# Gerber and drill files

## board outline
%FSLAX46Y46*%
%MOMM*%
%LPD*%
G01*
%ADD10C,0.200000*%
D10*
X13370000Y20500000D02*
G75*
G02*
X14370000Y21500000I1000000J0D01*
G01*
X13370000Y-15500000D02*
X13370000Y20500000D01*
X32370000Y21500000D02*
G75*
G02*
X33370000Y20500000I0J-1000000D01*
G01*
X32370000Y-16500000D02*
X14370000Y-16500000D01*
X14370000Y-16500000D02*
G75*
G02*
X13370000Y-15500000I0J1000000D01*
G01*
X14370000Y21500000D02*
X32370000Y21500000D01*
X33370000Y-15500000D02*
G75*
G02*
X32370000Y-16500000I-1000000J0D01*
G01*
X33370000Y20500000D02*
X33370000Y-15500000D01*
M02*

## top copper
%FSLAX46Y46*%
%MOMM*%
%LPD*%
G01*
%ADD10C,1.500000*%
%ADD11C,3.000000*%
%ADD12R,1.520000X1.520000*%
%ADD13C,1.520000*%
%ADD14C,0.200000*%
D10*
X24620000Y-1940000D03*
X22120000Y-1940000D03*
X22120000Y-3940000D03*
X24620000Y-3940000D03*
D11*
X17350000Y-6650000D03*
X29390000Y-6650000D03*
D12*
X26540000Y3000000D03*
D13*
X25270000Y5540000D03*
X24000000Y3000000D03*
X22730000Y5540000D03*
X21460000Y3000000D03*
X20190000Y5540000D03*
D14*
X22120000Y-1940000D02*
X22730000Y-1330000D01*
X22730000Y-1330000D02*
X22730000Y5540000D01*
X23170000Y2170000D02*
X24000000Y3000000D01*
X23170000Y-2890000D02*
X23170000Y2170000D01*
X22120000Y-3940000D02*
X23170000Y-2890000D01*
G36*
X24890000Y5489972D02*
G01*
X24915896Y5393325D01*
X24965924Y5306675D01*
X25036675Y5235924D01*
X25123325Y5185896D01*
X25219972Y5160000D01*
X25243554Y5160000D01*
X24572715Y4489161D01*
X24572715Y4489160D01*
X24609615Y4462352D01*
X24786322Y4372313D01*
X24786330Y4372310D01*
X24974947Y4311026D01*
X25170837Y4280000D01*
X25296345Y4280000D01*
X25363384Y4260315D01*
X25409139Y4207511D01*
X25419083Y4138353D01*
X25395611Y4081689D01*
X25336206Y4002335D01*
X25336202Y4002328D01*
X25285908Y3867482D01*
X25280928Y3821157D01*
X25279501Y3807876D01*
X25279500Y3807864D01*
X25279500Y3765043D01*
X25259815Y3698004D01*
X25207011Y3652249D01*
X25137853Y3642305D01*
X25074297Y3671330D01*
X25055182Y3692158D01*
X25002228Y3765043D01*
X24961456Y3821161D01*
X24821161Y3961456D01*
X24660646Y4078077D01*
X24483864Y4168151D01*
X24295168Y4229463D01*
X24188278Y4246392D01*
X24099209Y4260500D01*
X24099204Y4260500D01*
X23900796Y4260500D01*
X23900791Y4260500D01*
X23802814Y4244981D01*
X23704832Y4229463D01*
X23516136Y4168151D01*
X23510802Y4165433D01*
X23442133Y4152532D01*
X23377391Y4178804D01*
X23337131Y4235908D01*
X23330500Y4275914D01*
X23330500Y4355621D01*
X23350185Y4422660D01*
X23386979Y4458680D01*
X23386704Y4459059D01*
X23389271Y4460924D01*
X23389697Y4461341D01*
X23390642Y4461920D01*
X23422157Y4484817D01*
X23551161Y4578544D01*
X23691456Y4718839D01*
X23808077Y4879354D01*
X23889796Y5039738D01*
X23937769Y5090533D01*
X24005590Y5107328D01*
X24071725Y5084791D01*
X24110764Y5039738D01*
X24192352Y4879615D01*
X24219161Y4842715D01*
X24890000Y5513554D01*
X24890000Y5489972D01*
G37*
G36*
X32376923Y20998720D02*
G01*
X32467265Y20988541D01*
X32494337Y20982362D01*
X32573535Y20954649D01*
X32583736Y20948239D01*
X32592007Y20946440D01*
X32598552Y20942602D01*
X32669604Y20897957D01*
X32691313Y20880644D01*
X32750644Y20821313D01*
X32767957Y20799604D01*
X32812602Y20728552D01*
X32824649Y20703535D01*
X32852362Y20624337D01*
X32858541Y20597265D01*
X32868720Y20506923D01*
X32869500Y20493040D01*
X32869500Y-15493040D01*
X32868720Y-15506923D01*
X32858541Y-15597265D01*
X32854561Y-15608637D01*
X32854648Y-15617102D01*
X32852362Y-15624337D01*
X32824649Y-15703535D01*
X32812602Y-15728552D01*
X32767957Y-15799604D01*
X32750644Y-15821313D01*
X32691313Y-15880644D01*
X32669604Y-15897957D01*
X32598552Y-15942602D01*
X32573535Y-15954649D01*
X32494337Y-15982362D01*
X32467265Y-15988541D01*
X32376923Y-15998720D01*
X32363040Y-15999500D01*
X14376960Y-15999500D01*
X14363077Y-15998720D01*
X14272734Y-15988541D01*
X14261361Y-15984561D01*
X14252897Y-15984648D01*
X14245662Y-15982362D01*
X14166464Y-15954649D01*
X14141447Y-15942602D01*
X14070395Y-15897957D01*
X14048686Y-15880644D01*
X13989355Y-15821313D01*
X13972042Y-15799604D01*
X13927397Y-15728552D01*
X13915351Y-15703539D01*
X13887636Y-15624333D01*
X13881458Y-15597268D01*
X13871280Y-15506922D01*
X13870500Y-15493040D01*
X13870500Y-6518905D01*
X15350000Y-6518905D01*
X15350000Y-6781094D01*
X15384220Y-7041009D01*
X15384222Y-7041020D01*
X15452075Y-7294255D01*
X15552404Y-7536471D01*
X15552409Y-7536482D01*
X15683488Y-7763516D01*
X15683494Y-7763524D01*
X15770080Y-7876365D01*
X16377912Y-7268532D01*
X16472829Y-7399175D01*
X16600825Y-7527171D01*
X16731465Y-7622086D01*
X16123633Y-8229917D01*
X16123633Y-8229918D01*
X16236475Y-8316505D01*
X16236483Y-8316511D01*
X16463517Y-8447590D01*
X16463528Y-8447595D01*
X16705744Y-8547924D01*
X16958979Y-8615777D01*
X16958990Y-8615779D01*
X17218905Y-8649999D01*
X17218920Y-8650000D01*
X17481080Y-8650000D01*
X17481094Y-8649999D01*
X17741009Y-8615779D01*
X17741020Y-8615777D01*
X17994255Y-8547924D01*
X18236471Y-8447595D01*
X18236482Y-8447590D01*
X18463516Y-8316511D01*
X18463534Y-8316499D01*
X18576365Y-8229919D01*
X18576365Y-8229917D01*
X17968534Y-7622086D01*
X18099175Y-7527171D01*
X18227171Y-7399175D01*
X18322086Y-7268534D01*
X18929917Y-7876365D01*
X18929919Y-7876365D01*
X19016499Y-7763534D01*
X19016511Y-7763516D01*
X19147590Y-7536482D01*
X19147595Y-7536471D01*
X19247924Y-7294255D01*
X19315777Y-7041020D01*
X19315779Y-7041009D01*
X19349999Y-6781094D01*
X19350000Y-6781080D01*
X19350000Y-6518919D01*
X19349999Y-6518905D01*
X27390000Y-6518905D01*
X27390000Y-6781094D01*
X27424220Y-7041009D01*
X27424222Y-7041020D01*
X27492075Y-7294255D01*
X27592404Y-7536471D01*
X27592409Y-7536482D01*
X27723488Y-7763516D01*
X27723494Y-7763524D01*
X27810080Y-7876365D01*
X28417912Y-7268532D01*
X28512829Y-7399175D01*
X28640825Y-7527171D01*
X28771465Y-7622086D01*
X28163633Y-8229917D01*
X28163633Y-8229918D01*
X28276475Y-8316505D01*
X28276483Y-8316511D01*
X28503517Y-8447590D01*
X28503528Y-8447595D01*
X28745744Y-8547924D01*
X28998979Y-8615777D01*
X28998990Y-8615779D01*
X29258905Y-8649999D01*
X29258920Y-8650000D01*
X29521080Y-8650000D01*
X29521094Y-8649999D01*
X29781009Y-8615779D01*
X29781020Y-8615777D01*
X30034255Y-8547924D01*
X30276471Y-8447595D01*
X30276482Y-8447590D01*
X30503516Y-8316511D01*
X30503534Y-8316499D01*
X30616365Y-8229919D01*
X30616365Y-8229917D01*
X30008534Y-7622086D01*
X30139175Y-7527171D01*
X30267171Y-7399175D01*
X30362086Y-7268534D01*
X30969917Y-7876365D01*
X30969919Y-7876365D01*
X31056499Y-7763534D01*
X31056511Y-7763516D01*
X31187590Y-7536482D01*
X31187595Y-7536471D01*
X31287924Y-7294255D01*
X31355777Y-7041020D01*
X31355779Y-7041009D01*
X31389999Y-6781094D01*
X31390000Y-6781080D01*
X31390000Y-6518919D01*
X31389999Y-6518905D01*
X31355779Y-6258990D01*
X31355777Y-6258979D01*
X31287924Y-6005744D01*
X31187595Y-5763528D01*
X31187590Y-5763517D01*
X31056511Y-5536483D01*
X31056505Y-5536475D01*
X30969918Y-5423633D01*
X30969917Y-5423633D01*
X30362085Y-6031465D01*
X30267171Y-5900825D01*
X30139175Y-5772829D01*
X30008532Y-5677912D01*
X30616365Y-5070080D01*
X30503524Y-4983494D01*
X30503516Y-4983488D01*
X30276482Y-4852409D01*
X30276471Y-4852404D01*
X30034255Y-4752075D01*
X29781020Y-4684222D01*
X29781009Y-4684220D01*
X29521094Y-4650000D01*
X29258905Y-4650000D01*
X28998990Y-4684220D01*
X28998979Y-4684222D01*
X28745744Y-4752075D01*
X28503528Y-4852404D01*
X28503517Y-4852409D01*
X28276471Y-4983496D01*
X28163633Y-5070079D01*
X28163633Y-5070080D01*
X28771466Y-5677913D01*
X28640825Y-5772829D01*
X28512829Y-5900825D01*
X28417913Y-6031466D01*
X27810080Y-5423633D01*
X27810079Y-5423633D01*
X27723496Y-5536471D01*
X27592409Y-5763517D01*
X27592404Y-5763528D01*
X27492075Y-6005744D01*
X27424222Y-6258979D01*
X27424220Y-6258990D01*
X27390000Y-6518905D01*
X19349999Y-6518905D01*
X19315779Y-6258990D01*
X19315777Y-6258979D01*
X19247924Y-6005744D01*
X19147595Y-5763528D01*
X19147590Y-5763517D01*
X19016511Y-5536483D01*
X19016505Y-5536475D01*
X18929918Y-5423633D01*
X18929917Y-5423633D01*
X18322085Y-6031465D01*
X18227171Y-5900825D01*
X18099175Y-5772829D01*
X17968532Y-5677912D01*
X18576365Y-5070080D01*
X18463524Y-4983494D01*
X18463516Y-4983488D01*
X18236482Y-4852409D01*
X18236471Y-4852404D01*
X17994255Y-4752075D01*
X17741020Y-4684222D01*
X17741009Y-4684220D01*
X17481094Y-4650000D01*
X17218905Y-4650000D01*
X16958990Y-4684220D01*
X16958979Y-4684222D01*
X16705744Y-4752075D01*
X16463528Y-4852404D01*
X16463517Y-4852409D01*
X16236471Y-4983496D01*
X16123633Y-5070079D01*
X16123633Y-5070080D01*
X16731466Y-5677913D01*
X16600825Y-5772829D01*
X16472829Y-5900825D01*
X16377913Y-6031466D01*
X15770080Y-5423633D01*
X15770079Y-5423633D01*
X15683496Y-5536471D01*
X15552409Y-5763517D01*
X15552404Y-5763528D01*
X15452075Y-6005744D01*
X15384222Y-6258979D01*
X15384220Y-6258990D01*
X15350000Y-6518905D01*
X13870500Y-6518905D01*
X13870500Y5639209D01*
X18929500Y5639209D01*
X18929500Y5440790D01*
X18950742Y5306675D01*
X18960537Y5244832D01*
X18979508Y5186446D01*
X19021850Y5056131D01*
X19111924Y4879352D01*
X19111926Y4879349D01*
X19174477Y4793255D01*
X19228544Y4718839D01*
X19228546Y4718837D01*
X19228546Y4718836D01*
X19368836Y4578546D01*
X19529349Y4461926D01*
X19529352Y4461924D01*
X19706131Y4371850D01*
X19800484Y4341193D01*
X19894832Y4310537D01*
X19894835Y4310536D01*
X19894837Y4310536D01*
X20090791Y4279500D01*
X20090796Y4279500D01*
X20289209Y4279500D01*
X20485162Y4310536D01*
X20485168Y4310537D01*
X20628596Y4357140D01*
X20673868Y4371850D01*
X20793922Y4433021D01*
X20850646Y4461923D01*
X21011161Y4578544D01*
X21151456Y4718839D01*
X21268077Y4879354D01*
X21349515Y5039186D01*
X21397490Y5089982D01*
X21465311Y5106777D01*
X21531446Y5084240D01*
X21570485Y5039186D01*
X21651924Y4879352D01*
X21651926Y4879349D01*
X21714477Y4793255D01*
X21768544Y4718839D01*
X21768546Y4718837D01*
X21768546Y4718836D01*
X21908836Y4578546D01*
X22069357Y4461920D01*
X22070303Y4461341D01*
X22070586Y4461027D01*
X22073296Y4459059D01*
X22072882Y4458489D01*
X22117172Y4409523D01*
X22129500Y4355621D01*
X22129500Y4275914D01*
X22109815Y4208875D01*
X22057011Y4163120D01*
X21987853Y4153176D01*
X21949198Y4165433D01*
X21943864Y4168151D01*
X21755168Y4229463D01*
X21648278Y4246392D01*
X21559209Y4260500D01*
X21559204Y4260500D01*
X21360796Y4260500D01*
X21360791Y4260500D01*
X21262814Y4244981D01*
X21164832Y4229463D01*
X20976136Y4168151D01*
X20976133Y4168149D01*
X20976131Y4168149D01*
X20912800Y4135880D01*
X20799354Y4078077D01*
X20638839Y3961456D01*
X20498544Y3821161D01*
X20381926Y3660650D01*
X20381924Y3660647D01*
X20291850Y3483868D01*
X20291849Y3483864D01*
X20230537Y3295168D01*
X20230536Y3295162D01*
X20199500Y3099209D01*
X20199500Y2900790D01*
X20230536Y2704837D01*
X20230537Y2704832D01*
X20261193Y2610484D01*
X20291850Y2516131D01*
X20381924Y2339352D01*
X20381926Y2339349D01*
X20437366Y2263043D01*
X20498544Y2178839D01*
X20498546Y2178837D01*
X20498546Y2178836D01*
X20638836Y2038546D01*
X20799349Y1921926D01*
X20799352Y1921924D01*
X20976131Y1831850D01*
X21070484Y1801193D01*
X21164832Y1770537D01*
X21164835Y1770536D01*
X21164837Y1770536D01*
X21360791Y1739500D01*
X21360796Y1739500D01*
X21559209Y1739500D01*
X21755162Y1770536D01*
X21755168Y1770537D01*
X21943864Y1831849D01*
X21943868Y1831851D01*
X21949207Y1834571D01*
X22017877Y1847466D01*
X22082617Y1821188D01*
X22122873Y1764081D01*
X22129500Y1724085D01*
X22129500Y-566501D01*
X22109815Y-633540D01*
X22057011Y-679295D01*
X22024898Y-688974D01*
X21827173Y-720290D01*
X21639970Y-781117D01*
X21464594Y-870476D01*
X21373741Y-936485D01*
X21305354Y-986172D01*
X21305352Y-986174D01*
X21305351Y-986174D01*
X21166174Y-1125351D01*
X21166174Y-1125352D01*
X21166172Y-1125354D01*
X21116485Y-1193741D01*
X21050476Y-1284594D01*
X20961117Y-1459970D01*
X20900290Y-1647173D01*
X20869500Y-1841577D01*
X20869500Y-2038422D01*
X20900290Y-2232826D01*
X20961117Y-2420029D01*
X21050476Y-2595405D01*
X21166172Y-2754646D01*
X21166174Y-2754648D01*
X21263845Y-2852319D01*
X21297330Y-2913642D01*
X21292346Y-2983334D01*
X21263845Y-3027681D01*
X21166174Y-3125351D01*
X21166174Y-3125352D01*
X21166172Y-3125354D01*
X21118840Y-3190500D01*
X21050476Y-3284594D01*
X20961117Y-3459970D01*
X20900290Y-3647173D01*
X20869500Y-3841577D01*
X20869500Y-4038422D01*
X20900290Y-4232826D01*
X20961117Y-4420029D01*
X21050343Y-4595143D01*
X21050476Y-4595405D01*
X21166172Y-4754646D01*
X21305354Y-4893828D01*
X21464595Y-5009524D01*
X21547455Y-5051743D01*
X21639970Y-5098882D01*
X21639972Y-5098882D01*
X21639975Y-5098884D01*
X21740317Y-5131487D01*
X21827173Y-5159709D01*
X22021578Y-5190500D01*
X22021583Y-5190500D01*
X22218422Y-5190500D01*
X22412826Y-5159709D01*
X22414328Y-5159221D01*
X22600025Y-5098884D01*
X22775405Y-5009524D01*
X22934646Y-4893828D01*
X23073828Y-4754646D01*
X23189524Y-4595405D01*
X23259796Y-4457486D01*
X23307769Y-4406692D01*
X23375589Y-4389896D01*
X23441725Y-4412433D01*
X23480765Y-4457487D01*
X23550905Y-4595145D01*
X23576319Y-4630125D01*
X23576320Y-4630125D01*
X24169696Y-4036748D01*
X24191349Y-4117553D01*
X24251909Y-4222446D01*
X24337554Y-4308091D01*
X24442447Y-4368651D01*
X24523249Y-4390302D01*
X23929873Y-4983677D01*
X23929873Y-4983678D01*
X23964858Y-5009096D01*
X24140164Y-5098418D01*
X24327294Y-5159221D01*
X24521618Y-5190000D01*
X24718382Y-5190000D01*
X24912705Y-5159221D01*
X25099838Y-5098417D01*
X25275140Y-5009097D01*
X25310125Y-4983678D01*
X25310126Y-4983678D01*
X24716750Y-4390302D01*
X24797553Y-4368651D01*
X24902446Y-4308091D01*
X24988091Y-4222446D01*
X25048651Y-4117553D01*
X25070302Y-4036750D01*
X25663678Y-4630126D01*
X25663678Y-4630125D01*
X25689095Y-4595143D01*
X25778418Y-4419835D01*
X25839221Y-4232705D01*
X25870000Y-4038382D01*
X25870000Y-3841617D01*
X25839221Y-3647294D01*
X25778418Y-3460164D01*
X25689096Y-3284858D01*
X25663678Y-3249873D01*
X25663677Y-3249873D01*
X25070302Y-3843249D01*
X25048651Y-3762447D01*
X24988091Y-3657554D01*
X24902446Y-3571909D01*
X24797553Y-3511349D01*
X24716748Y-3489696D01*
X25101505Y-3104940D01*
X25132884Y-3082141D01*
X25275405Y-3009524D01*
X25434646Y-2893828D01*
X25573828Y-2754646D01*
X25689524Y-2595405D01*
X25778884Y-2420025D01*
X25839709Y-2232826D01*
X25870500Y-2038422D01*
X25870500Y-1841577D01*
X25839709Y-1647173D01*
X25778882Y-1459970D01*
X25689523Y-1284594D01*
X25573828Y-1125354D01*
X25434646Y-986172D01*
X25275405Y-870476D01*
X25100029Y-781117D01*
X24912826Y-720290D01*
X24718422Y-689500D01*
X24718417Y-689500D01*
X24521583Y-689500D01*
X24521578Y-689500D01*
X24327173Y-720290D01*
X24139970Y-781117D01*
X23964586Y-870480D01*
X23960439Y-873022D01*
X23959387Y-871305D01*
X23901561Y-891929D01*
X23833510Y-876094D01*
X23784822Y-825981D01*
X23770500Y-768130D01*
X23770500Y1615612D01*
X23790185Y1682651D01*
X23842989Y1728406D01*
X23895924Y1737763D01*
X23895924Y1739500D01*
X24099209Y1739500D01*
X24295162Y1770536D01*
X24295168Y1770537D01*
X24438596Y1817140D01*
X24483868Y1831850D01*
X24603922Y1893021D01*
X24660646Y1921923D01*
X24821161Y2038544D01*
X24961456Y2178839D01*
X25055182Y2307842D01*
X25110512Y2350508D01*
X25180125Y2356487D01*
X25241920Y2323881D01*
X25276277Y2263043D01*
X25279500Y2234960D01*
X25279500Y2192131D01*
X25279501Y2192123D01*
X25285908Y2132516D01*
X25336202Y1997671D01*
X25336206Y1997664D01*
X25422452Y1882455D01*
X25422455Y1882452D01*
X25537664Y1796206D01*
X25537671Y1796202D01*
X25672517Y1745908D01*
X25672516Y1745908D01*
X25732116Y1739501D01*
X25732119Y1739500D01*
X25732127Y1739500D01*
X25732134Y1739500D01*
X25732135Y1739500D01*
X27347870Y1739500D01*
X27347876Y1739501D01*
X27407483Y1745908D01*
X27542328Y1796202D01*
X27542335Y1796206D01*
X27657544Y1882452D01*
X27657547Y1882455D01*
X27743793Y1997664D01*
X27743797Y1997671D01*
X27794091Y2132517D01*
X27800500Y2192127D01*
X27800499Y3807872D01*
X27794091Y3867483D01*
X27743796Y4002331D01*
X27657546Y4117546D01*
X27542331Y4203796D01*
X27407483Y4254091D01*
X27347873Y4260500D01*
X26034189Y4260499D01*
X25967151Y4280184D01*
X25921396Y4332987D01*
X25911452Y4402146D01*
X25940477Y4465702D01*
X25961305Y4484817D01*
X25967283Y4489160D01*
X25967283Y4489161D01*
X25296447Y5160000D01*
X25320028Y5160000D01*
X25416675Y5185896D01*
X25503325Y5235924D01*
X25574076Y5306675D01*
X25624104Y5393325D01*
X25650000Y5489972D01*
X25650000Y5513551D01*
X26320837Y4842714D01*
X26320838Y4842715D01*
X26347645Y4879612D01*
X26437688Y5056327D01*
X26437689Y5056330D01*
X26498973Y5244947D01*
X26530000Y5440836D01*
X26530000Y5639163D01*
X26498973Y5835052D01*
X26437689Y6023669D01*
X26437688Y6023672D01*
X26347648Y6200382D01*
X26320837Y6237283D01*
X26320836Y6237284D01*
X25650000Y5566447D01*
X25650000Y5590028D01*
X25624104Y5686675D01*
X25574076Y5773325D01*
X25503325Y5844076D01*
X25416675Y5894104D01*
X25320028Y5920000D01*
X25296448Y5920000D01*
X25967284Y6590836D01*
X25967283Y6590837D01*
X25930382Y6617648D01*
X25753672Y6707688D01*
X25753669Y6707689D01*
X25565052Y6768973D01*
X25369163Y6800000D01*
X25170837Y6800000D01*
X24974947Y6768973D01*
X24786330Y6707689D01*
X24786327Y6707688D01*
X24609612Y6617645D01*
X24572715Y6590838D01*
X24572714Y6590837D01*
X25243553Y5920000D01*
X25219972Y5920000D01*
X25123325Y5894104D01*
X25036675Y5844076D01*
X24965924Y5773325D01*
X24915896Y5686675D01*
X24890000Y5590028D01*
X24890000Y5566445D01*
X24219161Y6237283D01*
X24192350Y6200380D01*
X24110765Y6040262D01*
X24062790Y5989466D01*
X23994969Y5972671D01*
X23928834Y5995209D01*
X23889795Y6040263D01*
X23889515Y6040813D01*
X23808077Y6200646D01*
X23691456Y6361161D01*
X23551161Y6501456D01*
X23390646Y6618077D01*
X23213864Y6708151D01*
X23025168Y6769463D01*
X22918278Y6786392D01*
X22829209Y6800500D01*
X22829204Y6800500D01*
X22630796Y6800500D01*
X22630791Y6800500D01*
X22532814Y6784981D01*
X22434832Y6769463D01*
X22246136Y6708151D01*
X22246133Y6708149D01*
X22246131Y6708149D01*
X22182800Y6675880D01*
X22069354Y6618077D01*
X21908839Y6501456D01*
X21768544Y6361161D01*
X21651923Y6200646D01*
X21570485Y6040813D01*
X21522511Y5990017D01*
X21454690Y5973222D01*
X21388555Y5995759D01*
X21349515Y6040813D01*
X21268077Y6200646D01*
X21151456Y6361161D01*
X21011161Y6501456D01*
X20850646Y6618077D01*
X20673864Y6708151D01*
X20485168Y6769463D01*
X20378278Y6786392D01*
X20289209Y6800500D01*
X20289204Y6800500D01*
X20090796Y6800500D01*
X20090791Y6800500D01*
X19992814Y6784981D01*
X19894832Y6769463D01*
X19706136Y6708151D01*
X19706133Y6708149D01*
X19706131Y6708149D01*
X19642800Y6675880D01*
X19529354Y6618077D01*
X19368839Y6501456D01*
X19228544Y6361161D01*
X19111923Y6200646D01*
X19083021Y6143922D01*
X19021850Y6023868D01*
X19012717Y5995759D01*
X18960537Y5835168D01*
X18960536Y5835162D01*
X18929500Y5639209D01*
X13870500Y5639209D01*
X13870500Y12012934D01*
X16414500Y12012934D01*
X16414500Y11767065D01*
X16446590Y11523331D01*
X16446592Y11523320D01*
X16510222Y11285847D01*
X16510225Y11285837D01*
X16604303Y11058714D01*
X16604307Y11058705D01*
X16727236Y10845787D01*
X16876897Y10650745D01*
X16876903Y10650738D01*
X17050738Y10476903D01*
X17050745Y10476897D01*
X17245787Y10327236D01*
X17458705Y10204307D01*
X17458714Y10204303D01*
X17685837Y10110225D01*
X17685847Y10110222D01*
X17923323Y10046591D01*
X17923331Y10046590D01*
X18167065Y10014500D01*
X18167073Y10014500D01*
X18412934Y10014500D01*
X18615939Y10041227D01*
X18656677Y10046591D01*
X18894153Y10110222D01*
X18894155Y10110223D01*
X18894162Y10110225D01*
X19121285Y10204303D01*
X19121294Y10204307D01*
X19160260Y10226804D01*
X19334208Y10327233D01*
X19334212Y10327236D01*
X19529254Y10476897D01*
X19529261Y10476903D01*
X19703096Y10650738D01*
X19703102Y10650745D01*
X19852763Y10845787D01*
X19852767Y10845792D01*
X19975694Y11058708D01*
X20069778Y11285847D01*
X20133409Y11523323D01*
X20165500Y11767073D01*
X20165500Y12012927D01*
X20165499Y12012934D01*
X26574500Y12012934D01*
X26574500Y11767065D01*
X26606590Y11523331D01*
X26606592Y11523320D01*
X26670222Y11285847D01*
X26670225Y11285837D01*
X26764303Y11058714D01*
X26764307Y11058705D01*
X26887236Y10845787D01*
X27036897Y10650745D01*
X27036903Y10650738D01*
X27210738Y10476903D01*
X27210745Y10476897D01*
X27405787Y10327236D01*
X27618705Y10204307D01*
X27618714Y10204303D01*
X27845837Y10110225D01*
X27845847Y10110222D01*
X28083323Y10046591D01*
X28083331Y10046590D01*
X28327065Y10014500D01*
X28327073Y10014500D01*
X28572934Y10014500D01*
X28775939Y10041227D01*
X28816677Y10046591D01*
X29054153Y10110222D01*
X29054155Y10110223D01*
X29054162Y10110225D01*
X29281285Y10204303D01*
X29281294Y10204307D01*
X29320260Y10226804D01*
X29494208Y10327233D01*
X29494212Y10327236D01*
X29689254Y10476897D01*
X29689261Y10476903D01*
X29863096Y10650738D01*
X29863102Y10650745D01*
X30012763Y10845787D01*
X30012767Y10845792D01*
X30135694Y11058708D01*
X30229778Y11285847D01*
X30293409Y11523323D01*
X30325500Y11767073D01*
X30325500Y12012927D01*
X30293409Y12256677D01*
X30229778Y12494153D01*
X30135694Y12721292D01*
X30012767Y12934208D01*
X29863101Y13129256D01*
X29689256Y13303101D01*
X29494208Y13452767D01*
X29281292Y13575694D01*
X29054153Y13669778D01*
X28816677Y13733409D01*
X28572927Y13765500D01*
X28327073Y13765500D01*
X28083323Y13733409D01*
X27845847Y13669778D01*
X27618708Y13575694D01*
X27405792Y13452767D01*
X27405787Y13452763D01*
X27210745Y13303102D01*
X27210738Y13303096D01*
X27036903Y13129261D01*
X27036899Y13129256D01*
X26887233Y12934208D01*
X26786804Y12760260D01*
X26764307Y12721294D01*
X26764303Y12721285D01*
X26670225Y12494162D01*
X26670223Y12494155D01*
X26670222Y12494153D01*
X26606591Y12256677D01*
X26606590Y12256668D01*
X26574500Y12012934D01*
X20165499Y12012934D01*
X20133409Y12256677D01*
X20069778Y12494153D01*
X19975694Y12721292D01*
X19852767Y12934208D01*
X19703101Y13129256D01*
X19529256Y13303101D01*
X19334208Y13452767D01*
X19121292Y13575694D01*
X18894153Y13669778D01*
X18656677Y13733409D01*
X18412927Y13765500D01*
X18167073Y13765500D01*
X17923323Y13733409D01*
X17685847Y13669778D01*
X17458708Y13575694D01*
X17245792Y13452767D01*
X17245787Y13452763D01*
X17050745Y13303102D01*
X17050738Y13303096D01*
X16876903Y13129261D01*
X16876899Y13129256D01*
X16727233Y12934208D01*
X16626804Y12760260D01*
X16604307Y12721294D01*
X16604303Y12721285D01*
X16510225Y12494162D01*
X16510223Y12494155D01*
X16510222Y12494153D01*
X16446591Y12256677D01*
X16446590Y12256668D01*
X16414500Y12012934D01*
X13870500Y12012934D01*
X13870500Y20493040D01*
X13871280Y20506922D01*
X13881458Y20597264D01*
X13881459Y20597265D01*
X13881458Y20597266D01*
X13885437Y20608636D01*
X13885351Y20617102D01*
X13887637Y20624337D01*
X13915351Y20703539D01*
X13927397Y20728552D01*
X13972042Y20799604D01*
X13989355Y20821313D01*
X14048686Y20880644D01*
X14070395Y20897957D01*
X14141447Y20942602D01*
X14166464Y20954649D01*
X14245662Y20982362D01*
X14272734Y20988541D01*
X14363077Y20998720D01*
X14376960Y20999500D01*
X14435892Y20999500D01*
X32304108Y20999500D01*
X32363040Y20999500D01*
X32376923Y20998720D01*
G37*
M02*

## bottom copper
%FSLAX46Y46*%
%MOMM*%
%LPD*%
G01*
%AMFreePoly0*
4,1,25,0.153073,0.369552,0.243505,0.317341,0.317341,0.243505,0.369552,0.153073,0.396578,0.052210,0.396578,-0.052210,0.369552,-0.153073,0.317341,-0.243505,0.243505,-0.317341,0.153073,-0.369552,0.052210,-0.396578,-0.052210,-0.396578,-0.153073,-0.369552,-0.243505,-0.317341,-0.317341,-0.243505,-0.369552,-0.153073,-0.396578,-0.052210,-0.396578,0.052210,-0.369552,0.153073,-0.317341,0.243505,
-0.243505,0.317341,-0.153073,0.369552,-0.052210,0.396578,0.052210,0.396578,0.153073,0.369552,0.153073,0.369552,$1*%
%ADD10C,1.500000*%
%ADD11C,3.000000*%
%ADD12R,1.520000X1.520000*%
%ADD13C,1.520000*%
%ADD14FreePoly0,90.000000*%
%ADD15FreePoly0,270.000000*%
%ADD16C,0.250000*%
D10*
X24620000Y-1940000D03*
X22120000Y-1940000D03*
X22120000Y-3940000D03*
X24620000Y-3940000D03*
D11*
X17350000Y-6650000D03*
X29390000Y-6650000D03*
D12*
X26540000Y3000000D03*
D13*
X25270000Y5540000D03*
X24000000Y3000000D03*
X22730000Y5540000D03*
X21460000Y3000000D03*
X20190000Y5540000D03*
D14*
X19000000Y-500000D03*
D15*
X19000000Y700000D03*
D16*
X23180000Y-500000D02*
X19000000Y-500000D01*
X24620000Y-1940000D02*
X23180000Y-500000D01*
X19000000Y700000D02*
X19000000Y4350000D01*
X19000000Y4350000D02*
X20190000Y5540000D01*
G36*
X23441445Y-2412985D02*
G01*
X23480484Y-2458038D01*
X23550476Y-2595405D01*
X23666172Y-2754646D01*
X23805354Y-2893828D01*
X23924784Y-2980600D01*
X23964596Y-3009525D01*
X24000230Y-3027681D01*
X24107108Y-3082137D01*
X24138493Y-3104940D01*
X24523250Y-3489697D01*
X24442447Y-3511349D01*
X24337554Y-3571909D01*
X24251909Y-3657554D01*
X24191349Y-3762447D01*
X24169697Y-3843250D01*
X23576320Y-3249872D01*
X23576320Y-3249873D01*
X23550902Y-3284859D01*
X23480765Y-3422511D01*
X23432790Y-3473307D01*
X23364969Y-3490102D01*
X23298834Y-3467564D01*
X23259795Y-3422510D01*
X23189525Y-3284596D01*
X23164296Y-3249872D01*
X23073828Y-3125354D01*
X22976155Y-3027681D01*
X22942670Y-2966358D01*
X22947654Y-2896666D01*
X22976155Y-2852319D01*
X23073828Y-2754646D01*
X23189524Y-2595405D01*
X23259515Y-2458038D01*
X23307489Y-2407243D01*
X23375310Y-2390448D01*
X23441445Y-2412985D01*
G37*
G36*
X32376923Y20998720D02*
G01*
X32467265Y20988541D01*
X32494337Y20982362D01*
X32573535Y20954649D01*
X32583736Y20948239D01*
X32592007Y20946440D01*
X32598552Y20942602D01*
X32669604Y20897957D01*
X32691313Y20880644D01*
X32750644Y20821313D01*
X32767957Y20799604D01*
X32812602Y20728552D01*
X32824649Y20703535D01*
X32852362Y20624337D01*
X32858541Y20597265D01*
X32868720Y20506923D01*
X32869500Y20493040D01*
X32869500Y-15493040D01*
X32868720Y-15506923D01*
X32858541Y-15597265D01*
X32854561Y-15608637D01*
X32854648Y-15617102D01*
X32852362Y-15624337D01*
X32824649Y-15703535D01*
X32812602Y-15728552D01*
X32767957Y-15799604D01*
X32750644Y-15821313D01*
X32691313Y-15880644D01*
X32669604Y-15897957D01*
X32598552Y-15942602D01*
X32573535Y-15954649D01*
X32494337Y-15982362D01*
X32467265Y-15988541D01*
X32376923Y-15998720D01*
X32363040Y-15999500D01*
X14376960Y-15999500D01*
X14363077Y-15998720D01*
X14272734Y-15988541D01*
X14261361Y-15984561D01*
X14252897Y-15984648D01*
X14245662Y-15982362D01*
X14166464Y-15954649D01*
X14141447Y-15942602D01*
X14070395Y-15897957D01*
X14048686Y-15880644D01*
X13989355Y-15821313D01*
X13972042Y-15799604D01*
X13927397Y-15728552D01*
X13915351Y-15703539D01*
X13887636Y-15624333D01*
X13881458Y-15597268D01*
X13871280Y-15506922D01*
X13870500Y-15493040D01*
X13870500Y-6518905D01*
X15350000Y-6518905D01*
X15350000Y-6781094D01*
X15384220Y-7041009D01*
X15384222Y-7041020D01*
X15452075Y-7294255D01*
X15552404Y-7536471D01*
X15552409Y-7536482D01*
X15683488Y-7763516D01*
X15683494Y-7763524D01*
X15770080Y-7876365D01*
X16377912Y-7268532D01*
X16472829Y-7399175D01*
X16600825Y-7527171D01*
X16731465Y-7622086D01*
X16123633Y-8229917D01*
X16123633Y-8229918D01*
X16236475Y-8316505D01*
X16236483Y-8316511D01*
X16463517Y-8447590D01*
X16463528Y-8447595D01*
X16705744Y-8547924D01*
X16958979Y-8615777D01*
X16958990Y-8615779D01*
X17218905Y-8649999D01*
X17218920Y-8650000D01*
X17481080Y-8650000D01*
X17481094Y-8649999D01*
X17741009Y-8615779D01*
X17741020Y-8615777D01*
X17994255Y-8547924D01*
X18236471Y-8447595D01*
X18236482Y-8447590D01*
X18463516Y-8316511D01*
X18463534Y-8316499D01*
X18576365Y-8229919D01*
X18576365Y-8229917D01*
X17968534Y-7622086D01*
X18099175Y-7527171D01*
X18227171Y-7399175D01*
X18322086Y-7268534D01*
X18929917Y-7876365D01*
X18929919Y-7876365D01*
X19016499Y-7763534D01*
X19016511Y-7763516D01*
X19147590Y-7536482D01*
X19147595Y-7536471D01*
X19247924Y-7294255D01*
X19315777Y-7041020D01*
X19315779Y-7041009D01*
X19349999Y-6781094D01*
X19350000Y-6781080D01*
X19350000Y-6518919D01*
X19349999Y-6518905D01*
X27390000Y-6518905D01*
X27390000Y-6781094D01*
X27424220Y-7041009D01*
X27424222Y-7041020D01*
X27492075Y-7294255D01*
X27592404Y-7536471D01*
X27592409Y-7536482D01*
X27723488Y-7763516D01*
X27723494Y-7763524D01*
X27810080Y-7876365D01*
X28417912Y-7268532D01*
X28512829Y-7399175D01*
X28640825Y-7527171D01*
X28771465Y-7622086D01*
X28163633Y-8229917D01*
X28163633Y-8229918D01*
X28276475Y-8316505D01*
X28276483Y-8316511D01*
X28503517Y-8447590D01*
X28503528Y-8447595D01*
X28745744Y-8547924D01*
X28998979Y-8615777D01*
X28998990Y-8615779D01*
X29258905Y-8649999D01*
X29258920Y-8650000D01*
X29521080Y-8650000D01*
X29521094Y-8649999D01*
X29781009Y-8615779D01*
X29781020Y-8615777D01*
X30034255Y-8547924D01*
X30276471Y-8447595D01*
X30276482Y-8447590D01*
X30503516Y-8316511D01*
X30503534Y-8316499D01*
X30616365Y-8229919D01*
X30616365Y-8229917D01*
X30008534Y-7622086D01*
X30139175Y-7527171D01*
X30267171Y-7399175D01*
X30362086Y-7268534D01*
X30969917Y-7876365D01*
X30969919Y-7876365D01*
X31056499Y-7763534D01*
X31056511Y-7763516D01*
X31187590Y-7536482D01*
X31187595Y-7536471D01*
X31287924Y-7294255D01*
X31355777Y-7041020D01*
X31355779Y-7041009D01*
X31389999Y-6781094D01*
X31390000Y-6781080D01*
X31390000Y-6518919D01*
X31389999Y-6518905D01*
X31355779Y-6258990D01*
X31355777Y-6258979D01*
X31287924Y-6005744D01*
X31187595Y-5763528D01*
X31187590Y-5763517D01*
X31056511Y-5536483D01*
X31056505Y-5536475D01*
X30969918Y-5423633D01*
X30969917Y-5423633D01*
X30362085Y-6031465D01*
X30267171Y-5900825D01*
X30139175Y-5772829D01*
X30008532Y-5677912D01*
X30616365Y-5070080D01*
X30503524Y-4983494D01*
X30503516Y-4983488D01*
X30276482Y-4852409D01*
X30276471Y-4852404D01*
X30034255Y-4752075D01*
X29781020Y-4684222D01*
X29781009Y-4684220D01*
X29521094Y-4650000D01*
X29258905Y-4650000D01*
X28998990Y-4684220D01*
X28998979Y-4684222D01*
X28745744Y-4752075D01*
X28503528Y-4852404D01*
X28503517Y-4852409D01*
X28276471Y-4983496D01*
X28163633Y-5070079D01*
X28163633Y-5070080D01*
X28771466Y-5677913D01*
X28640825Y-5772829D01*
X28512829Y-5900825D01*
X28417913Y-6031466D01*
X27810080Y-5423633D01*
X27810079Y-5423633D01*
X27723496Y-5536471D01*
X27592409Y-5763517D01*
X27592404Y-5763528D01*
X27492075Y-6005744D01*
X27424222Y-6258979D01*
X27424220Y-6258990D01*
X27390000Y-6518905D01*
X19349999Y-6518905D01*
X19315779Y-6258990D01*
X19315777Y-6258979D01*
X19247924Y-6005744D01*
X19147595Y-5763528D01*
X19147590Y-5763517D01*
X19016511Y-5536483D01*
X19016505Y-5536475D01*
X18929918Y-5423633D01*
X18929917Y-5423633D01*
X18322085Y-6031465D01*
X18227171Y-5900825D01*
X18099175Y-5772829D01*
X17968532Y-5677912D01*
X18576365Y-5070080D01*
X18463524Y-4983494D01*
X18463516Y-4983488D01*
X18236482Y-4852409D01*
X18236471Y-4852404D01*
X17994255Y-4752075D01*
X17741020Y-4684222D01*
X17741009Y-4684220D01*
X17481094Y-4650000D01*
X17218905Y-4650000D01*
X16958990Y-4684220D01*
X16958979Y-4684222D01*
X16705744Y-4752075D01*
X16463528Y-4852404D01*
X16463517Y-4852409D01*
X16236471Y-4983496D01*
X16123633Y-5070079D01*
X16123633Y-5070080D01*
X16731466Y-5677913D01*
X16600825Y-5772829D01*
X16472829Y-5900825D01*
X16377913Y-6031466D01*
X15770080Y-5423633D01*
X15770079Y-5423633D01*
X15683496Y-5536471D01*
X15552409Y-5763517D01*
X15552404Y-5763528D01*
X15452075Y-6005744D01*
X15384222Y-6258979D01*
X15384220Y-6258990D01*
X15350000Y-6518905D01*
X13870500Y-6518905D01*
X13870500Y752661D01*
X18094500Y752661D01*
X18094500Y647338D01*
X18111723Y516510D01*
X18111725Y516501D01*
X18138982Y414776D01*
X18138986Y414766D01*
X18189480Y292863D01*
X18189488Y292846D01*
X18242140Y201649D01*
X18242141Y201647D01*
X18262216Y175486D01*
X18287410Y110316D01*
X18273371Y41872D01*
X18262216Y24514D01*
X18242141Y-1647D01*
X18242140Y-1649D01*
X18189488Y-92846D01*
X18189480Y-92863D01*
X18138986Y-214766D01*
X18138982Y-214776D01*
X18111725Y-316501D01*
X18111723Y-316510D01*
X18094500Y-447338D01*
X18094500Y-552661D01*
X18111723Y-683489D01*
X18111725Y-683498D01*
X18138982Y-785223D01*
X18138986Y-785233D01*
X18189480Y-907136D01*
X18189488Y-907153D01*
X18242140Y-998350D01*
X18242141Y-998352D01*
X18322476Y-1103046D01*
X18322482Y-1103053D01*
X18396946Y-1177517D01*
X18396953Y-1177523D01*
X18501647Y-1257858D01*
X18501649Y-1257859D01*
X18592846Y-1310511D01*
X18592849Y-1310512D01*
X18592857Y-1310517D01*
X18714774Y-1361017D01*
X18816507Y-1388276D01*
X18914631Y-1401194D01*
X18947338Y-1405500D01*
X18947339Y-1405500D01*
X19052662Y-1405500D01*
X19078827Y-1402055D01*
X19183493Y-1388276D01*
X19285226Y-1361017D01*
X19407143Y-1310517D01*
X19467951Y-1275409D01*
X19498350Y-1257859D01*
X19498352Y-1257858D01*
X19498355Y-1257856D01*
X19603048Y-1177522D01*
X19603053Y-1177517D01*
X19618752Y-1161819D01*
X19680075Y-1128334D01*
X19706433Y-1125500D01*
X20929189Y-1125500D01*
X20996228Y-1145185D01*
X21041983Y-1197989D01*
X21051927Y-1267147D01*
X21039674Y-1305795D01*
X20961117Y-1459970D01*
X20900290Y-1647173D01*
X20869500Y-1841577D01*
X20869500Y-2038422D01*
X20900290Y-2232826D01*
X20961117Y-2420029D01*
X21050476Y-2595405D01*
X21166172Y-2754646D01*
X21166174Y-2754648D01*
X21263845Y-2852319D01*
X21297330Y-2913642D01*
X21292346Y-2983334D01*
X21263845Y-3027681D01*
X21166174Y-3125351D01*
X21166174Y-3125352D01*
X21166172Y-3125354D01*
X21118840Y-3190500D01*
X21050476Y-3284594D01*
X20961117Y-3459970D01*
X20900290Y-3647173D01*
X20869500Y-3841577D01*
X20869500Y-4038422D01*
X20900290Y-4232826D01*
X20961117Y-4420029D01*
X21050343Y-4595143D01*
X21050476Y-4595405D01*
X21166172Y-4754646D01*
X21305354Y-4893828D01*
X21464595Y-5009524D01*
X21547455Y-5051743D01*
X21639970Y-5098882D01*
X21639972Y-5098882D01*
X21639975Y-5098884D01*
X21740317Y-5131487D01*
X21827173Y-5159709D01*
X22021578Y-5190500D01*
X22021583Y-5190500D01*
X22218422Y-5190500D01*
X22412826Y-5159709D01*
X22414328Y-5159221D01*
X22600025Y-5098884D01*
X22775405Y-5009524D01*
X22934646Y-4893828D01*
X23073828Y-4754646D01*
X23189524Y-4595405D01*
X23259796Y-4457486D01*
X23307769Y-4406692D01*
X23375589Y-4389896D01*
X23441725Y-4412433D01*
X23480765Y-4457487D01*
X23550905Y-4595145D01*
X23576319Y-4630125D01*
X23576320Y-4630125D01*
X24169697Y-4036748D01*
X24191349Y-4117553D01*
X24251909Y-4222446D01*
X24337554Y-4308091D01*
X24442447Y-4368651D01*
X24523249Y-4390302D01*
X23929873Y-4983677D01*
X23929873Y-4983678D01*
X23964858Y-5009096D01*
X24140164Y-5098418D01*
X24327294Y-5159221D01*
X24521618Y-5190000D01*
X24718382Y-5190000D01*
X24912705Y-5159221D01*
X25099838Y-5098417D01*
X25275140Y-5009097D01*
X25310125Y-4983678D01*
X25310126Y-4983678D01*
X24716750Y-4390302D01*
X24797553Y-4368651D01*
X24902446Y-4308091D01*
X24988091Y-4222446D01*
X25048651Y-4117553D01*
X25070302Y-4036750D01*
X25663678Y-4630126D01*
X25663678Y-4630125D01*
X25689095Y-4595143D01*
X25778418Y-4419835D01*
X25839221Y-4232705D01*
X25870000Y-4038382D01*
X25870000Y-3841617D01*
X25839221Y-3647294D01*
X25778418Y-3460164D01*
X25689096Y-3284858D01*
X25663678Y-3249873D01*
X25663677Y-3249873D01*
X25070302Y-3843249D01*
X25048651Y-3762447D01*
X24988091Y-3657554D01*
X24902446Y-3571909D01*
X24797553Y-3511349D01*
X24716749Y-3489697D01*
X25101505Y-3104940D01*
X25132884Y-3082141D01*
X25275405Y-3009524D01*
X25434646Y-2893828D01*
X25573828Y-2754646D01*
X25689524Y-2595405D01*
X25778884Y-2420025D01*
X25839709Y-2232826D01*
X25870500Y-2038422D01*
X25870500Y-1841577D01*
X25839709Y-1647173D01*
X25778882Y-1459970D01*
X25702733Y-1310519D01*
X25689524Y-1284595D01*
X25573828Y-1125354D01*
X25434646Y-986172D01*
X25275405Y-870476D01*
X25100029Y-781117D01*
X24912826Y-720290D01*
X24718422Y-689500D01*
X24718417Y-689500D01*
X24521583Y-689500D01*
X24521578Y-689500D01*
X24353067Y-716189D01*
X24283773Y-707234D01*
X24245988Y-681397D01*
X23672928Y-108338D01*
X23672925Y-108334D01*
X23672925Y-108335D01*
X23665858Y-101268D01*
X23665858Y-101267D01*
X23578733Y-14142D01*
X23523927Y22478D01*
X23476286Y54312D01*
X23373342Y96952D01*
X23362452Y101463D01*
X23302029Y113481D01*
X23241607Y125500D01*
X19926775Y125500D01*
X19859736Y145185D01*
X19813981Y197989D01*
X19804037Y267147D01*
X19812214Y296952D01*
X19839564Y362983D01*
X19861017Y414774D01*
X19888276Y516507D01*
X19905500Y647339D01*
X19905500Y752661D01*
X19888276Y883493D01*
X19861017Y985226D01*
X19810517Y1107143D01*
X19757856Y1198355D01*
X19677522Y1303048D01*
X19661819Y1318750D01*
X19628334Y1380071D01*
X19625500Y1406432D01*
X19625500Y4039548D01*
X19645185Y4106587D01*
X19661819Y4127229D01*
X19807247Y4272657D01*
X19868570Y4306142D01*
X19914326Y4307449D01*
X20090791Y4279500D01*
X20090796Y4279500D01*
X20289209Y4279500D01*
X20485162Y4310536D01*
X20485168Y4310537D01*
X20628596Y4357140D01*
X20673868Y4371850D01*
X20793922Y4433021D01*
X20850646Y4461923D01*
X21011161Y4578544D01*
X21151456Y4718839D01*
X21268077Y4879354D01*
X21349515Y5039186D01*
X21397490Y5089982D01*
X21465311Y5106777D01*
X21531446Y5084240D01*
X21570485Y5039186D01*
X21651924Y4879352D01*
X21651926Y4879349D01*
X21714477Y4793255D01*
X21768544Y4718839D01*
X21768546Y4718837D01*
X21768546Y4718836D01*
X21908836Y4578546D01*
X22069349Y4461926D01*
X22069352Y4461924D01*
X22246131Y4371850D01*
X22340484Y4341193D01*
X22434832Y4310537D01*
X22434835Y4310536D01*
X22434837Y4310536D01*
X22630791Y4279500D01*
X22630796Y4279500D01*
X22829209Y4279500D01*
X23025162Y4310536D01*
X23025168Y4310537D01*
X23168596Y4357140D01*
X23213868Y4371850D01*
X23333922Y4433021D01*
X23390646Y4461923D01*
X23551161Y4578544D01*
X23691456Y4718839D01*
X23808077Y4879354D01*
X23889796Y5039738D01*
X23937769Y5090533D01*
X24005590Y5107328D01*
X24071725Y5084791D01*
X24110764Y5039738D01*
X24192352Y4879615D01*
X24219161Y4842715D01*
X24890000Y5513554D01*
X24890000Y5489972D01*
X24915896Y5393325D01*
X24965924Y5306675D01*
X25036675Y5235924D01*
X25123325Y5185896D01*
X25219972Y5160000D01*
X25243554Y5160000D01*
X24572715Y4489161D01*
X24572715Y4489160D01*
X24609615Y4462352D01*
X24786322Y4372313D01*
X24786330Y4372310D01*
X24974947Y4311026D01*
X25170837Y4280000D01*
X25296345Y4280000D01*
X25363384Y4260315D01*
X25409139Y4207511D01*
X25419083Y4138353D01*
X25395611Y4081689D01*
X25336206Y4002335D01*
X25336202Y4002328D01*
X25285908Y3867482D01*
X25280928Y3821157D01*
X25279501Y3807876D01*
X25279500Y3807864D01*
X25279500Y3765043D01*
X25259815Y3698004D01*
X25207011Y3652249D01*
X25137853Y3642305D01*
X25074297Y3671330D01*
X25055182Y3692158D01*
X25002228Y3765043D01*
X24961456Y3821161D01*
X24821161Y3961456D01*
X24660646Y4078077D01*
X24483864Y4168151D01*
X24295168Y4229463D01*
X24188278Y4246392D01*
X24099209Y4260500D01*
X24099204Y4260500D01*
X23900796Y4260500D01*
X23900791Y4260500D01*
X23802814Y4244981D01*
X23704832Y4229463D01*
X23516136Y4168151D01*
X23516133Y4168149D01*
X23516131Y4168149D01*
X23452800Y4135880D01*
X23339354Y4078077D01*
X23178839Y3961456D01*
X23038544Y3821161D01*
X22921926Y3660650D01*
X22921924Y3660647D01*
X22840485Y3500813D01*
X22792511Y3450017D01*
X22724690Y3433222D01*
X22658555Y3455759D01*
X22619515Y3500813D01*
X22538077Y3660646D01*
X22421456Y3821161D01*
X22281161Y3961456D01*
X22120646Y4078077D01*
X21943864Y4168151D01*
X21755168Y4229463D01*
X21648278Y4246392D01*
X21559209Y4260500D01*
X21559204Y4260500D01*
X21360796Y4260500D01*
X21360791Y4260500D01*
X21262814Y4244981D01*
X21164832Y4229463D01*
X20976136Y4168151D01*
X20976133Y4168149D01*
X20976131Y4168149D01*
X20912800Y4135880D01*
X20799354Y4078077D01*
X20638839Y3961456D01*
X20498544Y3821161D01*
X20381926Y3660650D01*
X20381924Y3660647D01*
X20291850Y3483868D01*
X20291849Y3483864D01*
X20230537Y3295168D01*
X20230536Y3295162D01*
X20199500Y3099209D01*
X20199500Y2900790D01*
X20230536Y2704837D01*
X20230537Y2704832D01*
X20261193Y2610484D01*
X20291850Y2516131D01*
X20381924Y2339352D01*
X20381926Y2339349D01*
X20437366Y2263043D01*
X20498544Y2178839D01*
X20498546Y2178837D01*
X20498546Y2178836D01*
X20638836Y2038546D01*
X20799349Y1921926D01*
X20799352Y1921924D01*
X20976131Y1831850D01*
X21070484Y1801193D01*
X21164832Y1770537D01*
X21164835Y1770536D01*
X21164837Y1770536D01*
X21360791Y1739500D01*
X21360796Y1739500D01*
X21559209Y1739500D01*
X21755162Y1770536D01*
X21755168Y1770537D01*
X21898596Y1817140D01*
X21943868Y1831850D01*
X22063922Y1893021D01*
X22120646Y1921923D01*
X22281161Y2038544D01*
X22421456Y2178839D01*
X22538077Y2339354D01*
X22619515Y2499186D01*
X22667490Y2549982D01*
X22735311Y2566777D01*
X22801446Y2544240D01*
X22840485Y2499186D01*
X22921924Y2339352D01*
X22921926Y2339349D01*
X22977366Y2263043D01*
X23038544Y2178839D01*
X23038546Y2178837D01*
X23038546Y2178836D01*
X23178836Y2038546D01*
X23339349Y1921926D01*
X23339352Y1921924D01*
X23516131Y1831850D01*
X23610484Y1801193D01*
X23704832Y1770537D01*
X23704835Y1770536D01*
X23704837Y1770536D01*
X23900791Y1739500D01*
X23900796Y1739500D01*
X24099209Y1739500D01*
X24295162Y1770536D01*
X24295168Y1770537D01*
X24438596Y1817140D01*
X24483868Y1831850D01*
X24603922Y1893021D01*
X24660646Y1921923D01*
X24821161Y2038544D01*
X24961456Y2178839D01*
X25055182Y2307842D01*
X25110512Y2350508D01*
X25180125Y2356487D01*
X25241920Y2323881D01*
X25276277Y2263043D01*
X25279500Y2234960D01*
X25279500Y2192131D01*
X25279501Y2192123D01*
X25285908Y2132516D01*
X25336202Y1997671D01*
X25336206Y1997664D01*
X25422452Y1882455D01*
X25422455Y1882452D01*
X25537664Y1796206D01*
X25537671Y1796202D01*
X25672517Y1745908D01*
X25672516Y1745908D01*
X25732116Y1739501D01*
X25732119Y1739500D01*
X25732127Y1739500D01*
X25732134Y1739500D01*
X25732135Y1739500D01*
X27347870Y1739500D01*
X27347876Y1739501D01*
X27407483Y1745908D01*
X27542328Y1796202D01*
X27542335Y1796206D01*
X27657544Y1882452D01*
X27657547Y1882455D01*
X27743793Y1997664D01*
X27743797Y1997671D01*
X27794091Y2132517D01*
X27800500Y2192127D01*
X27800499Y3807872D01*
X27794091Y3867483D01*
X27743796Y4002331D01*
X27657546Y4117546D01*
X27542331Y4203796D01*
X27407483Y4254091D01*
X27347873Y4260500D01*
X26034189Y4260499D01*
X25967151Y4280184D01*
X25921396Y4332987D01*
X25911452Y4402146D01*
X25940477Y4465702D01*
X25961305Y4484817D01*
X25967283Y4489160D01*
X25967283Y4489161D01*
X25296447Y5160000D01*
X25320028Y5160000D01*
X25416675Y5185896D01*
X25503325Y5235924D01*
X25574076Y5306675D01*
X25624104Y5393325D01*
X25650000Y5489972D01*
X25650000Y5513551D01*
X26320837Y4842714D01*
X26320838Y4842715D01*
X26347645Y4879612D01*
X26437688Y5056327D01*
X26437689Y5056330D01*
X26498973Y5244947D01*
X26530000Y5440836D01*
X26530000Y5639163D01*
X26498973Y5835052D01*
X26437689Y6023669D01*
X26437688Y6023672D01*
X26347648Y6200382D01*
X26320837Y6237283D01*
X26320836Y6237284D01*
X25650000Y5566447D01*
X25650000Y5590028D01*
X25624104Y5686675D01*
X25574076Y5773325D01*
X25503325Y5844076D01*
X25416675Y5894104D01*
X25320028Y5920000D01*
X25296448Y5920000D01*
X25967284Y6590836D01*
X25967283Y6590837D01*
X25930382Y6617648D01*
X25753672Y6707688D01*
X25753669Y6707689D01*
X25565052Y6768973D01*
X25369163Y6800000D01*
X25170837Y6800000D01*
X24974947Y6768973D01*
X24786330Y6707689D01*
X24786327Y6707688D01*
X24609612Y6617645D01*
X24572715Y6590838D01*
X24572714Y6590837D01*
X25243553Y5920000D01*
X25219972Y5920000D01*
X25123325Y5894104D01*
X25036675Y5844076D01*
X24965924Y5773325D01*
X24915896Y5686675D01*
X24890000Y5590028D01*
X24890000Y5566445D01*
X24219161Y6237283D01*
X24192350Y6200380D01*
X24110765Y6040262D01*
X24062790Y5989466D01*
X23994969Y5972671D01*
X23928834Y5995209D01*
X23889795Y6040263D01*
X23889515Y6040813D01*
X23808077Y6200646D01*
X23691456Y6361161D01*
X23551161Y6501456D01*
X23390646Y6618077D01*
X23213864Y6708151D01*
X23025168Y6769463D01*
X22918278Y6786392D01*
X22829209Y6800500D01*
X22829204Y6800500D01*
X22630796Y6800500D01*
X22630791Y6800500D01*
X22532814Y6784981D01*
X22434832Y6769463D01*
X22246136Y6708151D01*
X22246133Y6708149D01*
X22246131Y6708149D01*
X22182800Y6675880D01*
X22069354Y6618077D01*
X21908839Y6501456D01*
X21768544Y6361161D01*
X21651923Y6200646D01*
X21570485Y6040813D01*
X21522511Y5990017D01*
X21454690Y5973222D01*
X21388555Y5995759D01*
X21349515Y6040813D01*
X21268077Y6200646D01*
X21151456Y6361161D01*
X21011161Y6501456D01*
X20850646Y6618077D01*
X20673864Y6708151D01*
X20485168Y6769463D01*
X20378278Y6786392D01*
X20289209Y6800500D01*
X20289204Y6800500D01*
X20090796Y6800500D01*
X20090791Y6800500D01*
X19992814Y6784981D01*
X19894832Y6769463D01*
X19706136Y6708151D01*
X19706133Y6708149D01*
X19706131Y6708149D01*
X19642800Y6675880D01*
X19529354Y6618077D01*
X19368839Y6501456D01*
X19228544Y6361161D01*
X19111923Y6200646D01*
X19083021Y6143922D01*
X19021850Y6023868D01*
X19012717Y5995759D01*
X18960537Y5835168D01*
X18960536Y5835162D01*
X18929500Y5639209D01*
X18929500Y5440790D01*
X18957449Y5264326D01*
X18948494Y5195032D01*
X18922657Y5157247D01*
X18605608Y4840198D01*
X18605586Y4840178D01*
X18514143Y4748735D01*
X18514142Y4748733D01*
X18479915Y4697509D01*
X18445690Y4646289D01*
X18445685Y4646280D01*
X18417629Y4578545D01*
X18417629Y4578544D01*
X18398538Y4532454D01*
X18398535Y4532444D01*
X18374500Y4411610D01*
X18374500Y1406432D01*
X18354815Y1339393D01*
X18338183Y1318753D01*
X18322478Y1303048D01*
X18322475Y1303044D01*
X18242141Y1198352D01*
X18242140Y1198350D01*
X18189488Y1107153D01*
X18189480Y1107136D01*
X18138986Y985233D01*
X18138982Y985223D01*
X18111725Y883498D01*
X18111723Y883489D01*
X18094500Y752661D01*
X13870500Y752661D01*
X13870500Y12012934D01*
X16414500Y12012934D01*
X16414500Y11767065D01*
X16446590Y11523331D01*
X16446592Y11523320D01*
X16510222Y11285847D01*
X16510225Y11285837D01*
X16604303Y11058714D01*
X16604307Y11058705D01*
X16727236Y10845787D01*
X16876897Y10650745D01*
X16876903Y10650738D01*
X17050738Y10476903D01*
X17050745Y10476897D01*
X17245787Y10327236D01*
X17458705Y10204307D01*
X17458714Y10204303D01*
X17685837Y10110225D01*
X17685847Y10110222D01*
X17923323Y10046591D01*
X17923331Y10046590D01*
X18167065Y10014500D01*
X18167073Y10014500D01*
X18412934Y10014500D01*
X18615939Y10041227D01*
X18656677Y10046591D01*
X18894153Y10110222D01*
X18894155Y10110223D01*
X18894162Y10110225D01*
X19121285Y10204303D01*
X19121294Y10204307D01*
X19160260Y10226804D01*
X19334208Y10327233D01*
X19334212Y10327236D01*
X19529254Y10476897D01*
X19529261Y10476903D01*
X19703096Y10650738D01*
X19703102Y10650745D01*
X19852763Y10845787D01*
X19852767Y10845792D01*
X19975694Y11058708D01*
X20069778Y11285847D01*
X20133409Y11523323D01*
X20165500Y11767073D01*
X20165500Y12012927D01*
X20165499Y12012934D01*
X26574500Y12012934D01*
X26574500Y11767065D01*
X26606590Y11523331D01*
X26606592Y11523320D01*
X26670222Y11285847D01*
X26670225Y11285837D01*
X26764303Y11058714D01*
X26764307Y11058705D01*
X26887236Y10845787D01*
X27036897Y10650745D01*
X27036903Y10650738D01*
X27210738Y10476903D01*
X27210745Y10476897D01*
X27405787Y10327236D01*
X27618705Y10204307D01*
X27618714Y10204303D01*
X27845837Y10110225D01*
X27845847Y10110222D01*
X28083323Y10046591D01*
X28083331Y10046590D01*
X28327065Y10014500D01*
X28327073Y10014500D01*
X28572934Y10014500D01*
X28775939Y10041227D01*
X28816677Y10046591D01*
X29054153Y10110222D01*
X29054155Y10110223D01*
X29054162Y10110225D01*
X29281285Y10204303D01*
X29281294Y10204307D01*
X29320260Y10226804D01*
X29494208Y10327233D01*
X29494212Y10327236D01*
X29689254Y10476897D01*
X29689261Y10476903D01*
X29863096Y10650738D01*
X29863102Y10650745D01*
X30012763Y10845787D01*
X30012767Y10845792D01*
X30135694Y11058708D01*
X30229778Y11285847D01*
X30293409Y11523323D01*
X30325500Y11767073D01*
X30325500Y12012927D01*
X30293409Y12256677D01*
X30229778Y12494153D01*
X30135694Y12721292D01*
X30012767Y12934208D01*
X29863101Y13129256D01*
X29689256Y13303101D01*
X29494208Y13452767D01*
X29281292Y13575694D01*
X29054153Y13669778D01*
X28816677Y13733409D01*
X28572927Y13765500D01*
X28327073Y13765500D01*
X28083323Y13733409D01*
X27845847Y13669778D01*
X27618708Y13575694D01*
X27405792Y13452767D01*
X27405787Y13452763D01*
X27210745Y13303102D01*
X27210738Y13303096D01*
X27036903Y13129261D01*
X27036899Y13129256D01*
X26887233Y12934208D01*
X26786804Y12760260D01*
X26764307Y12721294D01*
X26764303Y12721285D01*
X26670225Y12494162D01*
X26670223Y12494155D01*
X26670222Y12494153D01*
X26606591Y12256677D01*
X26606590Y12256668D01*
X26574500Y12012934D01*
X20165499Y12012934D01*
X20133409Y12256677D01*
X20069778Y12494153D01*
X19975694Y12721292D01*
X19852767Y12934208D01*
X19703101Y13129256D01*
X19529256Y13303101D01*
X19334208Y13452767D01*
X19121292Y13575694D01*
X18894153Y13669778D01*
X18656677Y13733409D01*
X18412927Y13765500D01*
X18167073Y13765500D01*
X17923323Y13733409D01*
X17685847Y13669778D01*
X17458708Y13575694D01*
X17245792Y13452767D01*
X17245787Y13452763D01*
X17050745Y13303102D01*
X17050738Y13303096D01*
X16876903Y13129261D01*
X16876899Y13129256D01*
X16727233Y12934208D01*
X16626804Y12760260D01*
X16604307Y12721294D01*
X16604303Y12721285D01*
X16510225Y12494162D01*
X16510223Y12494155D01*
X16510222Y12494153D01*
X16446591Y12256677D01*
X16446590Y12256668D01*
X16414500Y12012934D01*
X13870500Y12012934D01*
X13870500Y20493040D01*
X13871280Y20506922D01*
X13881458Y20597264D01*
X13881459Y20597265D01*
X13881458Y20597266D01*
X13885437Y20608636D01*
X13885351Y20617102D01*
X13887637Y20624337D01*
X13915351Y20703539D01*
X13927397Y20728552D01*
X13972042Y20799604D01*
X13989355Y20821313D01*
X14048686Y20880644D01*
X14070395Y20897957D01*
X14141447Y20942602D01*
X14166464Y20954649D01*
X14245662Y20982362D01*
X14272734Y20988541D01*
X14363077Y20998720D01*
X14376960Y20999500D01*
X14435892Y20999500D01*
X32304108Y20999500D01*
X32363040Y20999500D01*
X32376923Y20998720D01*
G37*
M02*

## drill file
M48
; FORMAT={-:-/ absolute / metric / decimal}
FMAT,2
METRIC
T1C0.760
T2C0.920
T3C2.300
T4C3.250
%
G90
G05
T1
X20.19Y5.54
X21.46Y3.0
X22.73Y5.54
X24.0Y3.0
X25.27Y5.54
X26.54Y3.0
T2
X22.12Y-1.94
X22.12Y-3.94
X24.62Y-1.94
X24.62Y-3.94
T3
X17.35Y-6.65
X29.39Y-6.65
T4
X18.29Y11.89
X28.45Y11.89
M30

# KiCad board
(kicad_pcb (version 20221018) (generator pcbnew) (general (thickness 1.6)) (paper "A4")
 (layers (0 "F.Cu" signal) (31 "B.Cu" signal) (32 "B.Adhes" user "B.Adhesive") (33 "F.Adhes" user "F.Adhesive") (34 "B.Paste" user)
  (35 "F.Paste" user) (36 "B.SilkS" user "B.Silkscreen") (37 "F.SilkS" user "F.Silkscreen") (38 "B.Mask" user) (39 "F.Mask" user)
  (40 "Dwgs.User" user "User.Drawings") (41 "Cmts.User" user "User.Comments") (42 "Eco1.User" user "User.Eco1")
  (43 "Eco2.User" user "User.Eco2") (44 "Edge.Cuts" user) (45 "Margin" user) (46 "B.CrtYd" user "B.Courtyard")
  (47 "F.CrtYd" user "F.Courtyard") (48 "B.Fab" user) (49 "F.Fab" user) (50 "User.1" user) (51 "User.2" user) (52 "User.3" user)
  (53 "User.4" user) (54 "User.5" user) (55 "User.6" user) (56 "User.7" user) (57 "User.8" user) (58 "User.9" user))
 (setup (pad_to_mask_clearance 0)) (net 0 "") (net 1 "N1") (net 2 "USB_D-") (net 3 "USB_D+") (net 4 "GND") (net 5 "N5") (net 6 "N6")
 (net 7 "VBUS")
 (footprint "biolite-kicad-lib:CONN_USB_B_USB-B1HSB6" (layer "F.Cu") (at 23.37 6.65)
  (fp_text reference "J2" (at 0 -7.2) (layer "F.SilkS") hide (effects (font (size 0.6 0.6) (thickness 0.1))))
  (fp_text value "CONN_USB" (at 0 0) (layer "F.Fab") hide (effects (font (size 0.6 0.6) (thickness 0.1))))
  (pad "1" thru_hole circle (at 1.25 -4.71) (size 1.5 1.5) (drill 0.92) (layers "*.Cu" "*.Mask") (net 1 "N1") (solder_mask_margin 0.07))
  (pad "2" thru_hole circle (at -1.25 -4.71) (size 1.5 1.5) (drill 0.92) (layers "*.Cu" "*.Mask") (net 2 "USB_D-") (solder_mask_margin 0.07))
  (pad "3" thru_hole circle (at -1.25 -2.71) (size 1.5 1.5) (drill 0.92) (layers "*.Cu" "*.Mask") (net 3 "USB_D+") (solder_mask_margin 0.07))
  (pad "4" thru_hole circle (at 1.25 -2.71) (size 1.5 1.5) (drill 0.92) (layers "*.Cu" "*.Mask") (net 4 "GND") (solder_mask_margin 0.07))
  (pad "CASE" thru_hole circle (at -6.02 0) (size 3 3) (drill 2.3) (layers "*.Cu" "*.Mask") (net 4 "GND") (solder_mask_margin 0.07))
  (pad "CASE" thru_hole circle (at 6.02 0) (size 3 3) (drill 2.3) (layers "*.Cu" "*.Mask") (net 4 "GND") (solder_mask_margin 0.07)))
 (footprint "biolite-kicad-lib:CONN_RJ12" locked (layer "F.Cu") (at 26.54 -3 180)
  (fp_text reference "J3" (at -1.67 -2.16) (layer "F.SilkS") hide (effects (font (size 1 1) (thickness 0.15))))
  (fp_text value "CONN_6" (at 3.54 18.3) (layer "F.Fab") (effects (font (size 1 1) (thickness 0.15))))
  (pad "" np_thru_hole circle locked (at -1.91 8.89 180) (size 3.25 3.25) (drill 3.25) (layers "*.Cu" "*.Mask"))
  (pad "" np_thru_hole circle locked (at 8.25 8.89 180) (size 3.25 3.25) (drill 3.25) (layers "*.Cu" "*.Mask"))
  (pad "1" thru_hole rect locked (at 0 0 180) (size 1.52 1.52) (drill 0.76) (layers "*.Cu" "*.Mask") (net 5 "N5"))
  (pad "2" thru_hole circle locked (at 1.27 2.54 180) (size 1.52 1.52) (drill 0.76) (layers "*.Cu" "*.Mask") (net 4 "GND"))
  (pad "3" thru_hole circle locked (at 2.54 0 180) (size 1.52 1.52) (drill 0.76) (layers "*.Cu" "*.Mask") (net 3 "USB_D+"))
  (pad "4" thru_hole circle locked (at 3.81 2.54 180) (size 1.52 1.52) (drill 0.76) (layers "*.Cu" "*.Mask") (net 2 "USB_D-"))
  (pad "5" thru_hole circle locked (at 5.08 0 180) (size 1.52 1.52) (drill 0.76) (layers "*.Cu" "*.Mask") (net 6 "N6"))
  (pad "6" thru_hole circle locked (at 6.35 2.54 180) (size 1.52 1.52) (drill 0.76) (layers "*.Cu" "*.Mask") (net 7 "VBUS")))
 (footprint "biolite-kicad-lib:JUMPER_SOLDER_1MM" (layer "B.Cu") (at 19 -0.1 90)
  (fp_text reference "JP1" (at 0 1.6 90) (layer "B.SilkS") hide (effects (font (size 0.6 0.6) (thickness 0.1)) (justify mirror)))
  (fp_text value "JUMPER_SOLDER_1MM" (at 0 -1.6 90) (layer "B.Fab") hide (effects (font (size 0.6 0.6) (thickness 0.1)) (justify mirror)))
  (pad "1" smd custom (at -0.6 0 90) (size 0.8 0.8) (layers "B.Cu") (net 1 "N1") (zone_connect 0) (thermal_bridge_angle 45)
   (options (clearance outline) (anchor circle)) (primitives))
  (pad "2" smd custom (at 0.6 0 270) (size 0.8 0.8) (layers "B.Cu") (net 7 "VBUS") (zone_connect 0) (thermal_bridge_angle 45)
   (options (clearance outline) (anchor circle)) (primitives)))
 (gr_arc (start 13.37 -20.5) (mid 13.662893 -21.207107) (end 14.37 -21.5) (stroke (width 0.2) (type default)) (layer "Edge.Cuts"))
 (gr_line (start 13.37 15.5) (end 13.37 -20.5) (stroke (width 0.2) (type default)) (layer "Edge.Cuts"))
 (gr_arc (start 32.37 -21.5) (mid 33.077107 -21.207107) (end 33.37 -20.5) (stroke (width 0.2) (type default)) (layer "Edge.Cuts"))
 (gr_line (start 32.37 16.5) (end 14.37 16.5) (stroke (width 0.2) (type default)) (layer "Edge.Cuts"))
 (gr_arc (start 14.37 16.5) (mid 13.662893 16.207107) (end 13.37 15.5) (stroke (width 0.2) (type default)) (layer "Edge.Cuts"))
 (gr_line (start 14.37 -21.5) (end 32.37 -21.5) (stroke (width 0.2) (type default)) (layer "Edge.Cuts"))
 (gr_arc (start 33.37 15.5) (mid 33.077107 16.207107) (end 32.37 16.5) (stroke (width 0.2) (type default)) (layer "Edge.Cuts"))
 (gr_line (start 33.37 -20.5) (end 33.37 15.5) (stroke (width 0.2) (type default)) (layer "Edge.Cuts"))
 (segment (start 23.18 0.5) (end 19 0.5) (width 0.25) (layer "B.Cu") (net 1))
 (segment (start 24.62 1.94) (end 23.18 0.5) (width 0.25) (layer "B.Cu") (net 1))
 (segment (start 22.12 1.94) (end 22.73 1.33) (width 0.2) (layer "F.Cu") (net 2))
 (segment (start 22.73 1.33) (end 22.73 -5.54) (width 0.2) (layer "F.Cu") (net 2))
 (segment (start 23.17 -2.17) (end 24 -3) (width 0.2) (layer "F.Cu") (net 3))
 (segment (start 23.17 2.89) (end 23.17 -2.17) (width 0.2) (layer "F.Cu") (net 3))
 (segment (start 22.12 3.94) (end 23.17 2.89) (width 0.2) (layer "F.Cu") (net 3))
 (segment (start 19 -0.7) (end 19 -4.35) (width 0.25) (layer "B.Cu") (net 7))
 (segment (start 19 -4.35) (end 20.19 -5.54) (width 0.25) (layer "B.Cu") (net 7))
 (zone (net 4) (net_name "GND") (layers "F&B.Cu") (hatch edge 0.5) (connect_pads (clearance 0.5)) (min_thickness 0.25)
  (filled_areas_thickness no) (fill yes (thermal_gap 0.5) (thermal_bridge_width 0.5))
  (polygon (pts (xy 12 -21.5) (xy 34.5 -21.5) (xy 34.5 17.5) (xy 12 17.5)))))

